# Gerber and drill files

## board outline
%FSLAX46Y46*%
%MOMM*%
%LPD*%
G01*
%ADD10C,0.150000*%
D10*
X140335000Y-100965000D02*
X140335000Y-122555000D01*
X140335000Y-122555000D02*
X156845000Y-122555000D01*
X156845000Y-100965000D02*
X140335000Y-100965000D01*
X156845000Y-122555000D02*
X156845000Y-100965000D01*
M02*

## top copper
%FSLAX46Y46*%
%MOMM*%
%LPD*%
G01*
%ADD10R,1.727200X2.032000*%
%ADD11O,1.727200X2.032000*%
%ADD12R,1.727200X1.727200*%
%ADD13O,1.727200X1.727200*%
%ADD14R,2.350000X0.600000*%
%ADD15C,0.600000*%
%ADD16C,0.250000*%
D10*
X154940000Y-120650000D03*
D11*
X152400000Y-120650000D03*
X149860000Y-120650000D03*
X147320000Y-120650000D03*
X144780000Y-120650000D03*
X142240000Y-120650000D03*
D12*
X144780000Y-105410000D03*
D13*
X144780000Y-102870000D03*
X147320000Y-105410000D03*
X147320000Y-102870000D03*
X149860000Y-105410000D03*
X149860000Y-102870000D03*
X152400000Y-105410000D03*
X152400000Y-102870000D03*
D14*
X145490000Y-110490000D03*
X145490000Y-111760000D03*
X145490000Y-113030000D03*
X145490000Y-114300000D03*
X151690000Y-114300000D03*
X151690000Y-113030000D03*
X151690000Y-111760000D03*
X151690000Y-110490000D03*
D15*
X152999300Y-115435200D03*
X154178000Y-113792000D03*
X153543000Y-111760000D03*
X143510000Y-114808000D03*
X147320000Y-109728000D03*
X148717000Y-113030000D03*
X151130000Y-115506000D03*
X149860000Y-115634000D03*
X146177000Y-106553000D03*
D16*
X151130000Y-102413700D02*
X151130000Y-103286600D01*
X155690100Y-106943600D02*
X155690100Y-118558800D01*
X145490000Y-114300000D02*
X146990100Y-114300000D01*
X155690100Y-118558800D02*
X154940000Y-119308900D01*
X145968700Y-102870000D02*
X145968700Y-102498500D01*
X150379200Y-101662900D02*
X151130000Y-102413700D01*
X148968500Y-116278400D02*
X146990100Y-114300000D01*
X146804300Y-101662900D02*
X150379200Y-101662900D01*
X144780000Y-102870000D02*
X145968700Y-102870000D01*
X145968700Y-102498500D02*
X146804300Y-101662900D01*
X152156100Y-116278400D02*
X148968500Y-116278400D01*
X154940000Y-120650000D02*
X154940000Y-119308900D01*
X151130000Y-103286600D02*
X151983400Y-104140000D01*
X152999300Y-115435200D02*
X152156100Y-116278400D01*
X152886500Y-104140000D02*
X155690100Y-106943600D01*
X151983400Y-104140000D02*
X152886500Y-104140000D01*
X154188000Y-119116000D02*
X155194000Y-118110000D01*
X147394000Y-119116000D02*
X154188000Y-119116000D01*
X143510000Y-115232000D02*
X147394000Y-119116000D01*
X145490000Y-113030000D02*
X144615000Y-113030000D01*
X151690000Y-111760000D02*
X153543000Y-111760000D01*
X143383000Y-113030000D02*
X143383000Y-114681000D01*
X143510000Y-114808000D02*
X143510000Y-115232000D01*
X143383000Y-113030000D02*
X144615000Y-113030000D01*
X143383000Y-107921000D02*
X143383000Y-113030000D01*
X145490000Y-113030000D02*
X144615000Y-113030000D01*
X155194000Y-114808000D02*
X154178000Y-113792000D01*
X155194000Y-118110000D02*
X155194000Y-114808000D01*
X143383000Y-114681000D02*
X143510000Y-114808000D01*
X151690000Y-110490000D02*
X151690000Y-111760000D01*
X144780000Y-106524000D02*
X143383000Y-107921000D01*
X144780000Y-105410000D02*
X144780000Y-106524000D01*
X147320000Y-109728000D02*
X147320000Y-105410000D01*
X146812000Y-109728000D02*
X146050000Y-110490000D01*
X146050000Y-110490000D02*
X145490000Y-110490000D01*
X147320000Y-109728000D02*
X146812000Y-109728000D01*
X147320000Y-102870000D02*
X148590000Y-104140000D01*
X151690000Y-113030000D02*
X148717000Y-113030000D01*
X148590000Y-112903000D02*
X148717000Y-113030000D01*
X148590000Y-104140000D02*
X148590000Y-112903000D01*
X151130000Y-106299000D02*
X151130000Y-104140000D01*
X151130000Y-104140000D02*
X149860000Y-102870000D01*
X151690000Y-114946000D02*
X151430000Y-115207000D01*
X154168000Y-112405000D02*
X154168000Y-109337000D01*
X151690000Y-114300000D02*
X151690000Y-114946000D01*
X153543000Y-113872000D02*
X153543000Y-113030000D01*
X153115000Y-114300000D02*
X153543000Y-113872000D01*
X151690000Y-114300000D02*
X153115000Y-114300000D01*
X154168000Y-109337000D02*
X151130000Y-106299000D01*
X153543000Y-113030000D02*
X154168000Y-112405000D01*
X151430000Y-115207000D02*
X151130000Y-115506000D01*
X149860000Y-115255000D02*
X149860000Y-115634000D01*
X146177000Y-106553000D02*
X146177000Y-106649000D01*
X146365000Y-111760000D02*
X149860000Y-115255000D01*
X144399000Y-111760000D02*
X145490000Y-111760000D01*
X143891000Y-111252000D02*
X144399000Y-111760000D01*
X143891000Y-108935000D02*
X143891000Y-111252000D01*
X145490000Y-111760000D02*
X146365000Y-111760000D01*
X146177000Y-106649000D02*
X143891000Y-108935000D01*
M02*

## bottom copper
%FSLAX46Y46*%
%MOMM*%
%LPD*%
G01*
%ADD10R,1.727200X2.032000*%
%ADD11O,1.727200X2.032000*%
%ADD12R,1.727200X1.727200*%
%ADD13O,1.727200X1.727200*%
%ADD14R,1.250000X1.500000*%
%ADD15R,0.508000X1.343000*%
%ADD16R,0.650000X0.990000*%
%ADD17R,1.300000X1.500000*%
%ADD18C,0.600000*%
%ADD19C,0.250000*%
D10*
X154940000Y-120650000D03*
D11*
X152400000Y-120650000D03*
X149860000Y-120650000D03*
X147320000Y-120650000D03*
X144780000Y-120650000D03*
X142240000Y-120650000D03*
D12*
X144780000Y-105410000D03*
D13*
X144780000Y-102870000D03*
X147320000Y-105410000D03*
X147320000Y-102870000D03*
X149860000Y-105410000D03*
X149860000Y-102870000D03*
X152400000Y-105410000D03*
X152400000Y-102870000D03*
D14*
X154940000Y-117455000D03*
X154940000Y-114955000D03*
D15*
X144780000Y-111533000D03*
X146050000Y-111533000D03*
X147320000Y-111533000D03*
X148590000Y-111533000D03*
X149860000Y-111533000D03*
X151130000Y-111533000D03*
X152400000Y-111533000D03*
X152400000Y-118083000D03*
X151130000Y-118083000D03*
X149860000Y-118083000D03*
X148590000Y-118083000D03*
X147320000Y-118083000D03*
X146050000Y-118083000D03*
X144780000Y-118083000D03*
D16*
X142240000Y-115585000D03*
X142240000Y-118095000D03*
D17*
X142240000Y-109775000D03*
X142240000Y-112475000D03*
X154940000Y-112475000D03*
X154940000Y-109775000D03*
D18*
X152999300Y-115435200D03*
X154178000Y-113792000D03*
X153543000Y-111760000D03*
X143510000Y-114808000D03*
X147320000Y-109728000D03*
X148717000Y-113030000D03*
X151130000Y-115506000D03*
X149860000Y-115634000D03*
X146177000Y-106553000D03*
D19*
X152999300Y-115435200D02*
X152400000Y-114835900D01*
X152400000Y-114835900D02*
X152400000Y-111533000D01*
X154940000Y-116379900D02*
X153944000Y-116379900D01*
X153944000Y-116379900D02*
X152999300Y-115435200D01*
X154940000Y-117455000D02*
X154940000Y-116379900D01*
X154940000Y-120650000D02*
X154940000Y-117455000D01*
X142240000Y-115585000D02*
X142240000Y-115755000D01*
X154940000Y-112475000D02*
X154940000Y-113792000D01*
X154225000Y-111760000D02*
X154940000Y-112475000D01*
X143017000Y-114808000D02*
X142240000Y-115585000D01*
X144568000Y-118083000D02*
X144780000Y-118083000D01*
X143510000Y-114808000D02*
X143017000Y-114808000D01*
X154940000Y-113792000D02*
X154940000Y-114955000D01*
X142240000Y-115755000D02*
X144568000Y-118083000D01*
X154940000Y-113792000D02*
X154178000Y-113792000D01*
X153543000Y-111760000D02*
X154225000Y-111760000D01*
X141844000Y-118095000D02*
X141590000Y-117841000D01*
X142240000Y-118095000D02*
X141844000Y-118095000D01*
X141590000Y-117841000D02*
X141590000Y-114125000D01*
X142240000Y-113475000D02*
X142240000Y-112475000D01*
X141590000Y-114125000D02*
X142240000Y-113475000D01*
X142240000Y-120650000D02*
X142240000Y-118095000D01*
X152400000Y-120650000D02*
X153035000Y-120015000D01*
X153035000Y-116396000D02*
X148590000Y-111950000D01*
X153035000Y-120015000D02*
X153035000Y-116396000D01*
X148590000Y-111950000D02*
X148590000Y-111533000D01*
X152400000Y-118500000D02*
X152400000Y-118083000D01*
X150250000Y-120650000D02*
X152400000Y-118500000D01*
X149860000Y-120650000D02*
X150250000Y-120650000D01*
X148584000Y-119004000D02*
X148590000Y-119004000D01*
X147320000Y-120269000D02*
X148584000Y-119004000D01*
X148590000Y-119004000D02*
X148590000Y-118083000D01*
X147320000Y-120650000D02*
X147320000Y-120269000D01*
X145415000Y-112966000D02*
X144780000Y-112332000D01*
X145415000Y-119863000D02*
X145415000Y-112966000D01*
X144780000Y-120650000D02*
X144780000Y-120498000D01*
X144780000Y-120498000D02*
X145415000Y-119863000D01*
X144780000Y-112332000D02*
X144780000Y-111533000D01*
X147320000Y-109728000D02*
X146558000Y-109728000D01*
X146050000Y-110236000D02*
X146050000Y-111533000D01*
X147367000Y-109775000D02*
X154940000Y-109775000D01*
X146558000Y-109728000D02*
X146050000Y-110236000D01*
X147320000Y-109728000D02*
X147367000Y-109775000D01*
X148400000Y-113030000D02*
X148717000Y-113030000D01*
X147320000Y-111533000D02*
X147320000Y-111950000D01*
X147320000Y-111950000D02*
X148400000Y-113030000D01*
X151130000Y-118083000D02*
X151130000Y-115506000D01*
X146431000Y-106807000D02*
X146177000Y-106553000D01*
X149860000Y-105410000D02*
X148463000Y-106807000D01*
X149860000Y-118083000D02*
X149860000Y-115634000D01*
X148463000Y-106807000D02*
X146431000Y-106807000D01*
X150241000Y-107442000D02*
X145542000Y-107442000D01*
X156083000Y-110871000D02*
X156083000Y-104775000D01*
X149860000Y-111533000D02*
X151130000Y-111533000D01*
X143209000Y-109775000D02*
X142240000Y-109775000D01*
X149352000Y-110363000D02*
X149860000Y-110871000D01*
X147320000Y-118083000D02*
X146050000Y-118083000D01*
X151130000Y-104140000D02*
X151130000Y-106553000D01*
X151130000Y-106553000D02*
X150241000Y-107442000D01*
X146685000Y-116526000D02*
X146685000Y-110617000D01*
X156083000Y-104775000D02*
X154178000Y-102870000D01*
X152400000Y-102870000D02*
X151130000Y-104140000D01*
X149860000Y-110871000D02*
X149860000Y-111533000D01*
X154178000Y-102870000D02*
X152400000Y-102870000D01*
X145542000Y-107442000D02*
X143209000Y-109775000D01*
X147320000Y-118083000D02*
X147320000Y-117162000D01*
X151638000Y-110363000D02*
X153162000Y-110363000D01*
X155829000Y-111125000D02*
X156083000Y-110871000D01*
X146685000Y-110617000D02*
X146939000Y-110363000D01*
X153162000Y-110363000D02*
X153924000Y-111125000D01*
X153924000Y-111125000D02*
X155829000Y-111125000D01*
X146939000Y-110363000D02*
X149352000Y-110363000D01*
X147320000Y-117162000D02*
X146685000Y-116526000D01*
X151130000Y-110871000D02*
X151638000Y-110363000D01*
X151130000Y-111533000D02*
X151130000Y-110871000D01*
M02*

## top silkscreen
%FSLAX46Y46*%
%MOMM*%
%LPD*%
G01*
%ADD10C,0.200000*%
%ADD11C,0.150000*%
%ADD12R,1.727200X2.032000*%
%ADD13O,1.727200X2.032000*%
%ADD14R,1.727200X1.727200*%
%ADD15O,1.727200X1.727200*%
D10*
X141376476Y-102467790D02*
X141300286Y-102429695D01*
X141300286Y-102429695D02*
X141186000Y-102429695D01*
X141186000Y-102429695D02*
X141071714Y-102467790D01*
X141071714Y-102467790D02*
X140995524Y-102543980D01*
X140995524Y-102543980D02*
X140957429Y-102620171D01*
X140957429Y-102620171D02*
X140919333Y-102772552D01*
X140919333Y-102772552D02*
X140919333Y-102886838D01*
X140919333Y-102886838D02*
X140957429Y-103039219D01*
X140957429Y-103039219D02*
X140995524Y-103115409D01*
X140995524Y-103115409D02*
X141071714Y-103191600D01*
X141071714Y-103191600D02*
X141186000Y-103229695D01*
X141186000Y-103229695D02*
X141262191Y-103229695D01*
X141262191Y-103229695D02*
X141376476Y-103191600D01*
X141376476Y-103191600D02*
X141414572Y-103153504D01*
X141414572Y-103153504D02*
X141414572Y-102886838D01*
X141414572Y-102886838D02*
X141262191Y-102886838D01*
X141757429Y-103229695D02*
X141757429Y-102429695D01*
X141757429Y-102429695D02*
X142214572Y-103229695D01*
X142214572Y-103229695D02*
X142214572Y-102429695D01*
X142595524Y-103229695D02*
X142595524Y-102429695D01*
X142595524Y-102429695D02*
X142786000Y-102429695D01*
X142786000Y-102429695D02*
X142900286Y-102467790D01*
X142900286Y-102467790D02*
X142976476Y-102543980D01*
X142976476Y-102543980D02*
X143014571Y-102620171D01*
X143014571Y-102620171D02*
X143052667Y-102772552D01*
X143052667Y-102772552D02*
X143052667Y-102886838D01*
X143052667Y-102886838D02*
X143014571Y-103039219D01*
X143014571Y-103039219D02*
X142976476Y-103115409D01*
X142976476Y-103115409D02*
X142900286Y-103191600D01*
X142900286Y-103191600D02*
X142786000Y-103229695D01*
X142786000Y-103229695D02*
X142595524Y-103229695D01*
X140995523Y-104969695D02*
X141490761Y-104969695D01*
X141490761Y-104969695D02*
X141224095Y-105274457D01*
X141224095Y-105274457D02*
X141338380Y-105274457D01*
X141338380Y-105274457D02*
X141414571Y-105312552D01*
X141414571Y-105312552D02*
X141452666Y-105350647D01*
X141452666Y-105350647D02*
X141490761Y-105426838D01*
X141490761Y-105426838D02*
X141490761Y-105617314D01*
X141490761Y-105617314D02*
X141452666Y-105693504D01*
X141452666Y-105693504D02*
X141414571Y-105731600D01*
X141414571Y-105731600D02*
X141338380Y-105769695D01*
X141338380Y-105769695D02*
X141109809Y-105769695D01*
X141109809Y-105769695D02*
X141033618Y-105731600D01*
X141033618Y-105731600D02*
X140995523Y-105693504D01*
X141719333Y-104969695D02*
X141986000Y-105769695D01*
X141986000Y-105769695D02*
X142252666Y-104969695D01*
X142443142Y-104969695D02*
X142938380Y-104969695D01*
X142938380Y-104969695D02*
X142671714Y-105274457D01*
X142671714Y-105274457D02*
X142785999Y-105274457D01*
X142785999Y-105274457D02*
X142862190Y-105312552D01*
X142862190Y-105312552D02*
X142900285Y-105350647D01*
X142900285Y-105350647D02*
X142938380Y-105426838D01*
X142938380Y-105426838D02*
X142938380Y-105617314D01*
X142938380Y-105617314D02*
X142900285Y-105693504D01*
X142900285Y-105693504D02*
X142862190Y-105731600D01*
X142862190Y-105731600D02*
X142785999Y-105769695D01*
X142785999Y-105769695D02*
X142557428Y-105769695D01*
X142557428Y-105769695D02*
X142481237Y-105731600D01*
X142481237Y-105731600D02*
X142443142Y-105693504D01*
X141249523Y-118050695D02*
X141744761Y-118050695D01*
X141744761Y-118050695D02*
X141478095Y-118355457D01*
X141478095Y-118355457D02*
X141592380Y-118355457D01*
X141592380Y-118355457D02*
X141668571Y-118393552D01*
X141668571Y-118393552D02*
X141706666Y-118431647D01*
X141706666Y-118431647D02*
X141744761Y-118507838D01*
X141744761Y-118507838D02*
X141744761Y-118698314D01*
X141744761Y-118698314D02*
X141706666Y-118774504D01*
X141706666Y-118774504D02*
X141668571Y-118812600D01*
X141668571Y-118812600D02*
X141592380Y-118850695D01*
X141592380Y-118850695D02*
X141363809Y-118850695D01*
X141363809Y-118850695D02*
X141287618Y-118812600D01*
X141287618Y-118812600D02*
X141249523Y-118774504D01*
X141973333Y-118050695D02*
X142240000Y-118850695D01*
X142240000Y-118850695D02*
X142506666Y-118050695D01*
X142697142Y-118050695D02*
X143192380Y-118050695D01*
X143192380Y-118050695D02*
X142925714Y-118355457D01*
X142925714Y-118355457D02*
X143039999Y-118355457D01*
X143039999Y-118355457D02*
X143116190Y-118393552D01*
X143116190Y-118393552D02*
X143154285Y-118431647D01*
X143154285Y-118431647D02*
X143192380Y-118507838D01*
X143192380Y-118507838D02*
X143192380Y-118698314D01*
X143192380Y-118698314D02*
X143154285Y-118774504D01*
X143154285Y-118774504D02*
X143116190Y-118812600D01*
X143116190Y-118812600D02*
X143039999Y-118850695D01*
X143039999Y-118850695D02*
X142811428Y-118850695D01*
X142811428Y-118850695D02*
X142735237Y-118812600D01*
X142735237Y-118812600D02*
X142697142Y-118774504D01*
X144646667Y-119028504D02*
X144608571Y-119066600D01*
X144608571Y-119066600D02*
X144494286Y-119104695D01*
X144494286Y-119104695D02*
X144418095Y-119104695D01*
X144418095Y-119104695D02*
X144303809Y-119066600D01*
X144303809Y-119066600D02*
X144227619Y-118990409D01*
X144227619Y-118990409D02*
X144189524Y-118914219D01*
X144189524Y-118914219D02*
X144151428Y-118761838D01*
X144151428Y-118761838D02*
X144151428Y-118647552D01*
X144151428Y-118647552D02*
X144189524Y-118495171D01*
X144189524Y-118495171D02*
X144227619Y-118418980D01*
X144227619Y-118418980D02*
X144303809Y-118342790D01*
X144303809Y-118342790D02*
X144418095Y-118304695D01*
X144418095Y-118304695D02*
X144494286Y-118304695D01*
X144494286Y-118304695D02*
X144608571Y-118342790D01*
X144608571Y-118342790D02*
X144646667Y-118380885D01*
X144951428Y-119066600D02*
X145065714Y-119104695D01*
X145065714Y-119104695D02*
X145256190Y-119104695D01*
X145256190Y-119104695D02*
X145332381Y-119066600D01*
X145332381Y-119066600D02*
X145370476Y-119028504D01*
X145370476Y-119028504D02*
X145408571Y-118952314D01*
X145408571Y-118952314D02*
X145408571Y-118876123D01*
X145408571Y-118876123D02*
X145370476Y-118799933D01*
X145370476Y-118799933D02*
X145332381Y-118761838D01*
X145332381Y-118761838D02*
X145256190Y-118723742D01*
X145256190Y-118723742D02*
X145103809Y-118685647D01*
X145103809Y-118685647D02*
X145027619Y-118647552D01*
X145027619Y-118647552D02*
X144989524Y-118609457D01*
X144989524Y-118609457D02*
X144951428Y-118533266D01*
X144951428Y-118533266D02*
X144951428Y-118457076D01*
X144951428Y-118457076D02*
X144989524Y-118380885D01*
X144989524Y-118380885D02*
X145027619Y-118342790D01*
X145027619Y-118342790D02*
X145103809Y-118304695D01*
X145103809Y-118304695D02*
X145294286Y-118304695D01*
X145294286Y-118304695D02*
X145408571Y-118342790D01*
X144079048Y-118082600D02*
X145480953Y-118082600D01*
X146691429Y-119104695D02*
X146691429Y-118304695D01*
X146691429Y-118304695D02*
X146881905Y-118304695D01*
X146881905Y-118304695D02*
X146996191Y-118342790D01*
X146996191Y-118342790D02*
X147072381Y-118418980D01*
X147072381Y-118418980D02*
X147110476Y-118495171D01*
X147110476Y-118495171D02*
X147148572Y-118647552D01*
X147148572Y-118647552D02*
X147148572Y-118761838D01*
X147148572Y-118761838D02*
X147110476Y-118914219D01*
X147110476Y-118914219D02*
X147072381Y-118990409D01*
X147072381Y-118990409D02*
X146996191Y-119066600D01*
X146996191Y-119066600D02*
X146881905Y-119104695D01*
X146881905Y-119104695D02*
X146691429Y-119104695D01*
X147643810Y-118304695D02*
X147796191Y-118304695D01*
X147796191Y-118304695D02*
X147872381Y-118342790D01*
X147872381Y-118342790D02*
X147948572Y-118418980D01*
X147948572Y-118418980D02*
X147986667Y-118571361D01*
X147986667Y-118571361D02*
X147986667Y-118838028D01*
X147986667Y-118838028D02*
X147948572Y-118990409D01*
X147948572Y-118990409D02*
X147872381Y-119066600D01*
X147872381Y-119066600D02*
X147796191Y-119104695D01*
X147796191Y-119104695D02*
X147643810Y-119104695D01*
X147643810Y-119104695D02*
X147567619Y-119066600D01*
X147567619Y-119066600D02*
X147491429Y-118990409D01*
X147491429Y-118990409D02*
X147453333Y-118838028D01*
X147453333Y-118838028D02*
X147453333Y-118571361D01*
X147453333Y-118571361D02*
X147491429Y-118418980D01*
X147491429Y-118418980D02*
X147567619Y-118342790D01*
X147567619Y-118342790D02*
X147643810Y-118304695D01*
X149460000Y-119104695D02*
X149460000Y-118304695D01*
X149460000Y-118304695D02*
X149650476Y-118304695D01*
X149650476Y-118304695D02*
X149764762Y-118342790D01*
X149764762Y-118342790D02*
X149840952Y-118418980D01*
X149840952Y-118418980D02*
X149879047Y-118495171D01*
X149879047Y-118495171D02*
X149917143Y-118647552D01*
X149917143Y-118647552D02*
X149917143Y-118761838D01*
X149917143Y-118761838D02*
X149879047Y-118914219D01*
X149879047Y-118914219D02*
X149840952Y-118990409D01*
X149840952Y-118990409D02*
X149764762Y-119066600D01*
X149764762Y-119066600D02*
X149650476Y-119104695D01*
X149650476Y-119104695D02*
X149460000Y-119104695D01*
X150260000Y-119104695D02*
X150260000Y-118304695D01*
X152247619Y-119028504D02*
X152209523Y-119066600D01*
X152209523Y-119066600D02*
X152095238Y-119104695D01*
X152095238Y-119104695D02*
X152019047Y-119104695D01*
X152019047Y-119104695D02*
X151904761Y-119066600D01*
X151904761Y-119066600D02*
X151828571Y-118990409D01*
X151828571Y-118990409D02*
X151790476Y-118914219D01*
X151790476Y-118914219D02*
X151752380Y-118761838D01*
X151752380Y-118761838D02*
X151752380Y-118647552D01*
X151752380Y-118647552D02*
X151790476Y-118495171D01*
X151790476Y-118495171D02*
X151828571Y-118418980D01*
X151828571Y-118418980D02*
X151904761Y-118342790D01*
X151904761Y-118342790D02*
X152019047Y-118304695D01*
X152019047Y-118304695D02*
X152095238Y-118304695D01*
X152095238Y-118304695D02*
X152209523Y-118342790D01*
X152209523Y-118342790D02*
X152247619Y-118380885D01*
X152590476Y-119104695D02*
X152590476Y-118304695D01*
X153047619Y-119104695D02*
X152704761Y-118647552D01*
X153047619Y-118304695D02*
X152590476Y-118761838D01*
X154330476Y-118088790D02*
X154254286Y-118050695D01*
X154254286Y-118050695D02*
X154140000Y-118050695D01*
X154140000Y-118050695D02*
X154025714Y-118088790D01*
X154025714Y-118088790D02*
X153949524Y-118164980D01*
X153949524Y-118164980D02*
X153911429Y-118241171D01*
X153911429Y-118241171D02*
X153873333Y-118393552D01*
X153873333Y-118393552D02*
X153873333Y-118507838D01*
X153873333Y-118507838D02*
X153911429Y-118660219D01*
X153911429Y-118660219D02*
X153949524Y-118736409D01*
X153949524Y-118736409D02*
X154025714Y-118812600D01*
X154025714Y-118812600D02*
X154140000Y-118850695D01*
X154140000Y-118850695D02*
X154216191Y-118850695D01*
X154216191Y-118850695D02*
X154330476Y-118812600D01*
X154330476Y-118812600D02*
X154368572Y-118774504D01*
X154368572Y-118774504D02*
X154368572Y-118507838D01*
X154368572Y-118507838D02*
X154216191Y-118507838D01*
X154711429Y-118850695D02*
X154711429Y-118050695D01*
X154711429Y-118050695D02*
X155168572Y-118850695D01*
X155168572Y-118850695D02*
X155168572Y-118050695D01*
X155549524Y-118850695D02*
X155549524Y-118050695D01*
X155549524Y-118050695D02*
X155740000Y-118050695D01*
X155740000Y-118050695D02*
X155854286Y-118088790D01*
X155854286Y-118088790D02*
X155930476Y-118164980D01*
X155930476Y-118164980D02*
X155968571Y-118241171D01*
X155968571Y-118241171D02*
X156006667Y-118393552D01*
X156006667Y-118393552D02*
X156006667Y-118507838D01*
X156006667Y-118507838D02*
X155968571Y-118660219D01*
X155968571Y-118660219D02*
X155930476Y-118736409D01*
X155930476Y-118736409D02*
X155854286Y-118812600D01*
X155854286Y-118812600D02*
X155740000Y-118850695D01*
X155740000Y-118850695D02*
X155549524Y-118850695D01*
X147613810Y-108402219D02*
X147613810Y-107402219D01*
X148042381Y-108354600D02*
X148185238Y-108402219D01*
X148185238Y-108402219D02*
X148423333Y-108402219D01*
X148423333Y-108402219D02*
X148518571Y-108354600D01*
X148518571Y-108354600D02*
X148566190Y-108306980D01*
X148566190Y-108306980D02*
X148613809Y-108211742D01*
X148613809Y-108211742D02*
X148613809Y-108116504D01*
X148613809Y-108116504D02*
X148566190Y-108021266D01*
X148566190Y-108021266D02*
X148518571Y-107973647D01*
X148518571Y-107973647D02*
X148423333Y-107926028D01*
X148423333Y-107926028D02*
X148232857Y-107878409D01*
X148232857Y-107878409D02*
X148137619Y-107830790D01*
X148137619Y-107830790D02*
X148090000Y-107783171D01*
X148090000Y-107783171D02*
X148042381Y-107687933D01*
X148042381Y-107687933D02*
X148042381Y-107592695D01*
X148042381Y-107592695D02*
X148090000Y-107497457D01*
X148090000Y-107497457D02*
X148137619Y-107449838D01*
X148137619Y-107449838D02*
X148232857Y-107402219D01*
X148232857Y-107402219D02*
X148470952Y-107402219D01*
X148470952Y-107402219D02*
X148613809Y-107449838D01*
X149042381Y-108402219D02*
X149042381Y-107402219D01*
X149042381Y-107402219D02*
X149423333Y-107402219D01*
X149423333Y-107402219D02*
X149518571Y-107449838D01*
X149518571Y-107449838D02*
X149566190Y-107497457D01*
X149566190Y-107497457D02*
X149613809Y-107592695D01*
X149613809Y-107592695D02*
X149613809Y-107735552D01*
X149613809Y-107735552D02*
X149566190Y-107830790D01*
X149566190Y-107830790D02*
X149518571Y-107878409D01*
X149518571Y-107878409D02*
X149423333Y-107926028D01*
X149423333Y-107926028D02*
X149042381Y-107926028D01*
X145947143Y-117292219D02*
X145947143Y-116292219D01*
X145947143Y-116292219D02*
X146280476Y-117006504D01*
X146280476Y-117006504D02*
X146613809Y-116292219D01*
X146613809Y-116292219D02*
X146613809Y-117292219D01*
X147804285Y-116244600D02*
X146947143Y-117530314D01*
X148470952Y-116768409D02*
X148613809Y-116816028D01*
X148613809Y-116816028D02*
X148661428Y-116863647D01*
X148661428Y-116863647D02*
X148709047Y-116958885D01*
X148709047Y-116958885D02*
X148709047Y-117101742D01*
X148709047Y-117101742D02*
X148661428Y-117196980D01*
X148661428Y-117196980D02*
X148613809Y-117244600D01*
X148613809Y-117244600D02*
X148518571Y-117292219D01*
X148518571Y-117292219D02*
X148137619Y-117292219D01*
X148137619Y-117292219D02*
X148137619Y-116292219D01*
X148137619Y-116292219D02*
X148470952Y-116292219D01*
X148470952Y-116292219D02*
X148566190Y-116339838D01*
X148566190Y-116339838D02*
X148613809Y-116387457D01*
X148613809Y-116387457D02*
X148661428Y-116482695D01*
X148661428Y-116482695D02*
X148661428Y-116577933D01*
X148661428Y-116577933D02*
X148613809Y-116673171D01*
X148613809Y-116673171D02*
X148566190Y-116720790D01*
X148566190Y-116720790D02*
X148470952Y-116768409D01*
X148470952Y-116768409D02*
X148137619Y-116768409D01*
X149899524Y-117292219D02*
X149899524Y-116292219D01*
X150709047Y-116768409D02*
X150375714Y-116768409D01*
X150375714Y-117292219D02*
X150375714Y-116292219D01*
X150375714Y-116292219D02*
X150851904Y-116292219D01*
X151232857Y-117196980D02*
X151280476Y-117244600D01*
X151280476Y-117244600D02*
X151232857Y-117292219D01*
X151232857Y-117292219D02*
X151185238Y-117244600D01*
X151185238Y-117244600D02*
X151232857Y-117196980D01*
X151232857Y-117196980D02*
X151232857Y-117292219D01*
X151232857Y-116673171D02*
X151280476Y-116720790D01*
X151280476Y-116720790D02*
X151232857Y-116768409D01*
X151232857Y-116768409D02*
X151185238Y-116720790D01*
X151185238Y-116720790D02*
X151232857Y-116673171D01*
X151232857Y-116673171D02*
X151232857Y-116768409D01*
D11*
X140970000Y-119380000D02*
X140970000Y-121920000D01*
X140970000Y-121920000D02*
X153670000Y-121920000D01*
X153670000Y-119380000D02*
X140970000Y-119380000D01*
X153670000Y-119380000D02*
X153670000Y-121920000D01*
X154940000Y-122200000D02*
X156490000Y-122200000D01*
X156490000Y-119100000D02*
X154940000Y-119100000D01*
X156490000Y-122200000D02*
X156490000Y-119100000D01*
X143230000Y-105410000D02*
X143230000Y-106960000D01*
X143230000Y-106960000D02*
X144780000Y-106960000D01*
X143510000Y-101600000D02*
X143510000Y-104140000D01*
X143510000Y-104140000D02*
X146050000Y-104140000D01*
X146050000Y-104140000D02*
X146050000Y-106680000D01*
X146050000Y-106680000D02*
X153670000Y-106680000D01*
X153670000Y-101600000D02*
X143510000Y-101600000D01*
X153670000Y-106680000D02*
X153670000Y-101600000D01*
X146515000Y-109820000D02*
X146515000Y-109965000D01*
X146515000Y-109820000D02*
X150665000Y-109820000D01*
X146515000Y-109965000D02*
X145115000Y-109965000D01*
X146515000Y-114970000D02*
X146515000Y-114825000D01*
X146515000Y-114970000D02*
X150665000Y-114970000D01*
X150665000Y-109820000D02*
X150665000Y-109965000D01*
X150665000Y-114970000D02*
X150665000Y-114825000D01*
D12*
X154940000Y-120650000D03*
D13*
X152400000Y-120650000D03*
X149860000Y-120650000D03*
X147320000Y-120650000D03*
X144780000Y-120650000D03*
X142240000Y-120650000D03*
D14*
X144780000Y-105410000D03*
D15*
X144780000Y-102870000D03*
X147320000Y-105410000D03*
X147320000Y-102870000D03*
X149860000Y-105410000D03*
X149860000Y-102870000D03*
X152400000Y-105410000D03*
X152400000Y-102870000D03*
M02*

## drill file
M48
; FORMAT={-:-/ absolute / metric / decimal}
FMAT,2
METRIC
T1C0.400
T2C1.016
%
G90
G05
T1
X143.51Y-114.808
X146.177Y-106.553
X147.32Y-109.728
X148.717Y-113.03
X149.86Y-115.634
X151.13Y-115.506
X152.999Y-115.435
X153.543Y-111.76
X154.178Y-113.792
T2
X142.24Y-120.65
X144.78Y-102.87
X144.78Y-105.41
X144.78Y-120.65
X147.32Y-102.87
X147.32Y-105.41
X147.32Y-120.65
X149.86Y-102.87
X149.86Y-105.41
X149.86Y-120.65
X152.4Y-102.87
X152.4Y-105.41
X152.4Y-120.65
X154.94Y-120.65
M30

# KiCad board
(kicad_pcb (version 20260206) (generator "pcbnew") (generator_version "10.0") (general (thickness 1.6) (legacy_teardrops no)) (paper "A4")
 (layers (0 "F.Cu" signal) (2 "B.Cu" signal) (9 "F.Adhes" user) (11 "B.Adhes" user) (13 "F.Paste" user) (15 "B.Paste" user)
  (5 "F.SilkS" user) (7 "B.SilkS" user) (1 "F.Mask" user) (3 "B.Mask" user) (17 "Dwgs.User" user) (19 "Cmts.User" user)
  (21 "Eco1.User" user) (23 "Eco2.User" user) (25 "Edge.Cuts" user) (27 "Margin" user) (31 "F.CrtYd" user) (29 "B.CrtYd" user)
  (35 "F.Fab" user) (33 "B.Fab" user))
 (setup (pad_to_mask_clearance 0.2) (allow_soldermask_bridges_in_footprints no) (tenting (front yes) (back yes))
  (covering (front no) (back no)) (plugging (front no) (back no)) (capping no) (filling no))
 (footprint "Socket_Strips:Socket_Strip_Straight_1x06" (layer "F.Cu") (at 154.94 120.65 180)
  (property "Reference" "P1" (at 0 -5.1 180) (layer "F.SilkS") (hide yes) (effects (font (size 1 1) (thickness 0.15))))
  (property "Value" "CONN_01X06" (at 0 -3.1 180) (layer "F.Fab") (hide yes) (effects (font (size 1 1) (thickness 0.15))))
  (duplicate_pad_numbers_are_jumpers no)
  (fp_line (start 13.97 1.27) (end 13.97 -1.27) (stroke (width 0.15) (type solid)) (layer "F.SilkS"))
  (fp_line (start 13.97 -1.27) (end 1.27 -1.27) (stroke (width 0.15) (type solid)) (layer "F.SilkS"))
  (fp_line (start 1.27 1.27) (end 13.97 1.27) (stroke (width 0.15) (type solid)) (layer "F.SilkS"))
  (fp_line (start 1.27 1.27) (end 1.27 -1.27) (stroke (width 0.15) (type solid)) (layer "F.SilkS"))
  (fp_line (start 0 -1.55) (end -1.55 -1.55) (stroke (width 0.15) (type solid)) (layer "F.SilkS"))
  (fp_line (start -1.55 1.55) (end 0 1.55) (stroke (width 0.15) (type solid)) (layer "F.SilkS"))
  (fp_line (start -1.55 -1.55) (end -1.55 1.55) (stroke (width 0.15) (type solid)) (layer "F.SilkS"))
  (pad "1" thru_hole rect (at 0 0 180) (size 1.7272 2.032) (drill 1.016) (layers "*.Cu" "*.Mask" "F.SilkS") (remove_unused_layers no)
   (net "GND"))
  (pad "2" thru_hole oval (at 2.54 0 180) (size 1.7272 2.032) (drill 1.016) (layers "*.Cu" "*.Mask" "F.SilkS") (remove_unused_layers no)
   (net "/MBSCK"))
  (pad "3" thru_hole oval (at 5.08 0 180) (size 1.7272 2.032) (drill 1.016) (layers "*.Cu" "*.Mask" "F.SilkS") (remove_unused_layers no)
   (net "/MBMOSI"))
  (pad "4" thru_hole oval (at 7.62 0 180) (size 1.7272 2.032) (drill 1.016) (layers "*.Cu" "*.Mask" "F.SilkS") (remove_unused_layers no)
   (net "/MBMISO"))
  (pad "5" thru_hole oval (at 10.16 0 180) (size 1.7272 2.032) (drill 1.016) (layers "*.Cu" "*.Mask" "F.SilkS") (remove_unused_layers no)
   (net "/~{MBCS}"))
  (pad "6" thru_hole oval (at 12.7 0 180) (size 1.7272 2.032) (drill 1.016) (layers "*.Cu" "*.Mask" "F.SilkS") (remove_unused_layers no)
   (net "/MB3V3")))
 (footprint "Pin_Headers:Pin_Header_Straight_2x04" (layer "F.Cu") (at 144.78 105.41 90)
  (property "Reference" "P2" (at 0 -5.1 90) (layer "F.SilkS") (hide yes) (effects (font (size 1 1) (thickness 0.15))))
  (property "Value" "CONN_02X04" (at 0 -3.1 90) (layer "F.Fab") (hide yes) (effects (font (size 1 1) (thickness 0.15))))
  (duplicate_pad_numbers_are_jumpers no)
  (fp_line (start 0 -1.55) (end -1.55 -1.55) (stroke (width 0.15) (type solid)) (layer "F.SilkS"))
  (fp_line (start -1.55 -1.55) (end -1.55 0) (stroke (width 0.15) (type solid)) (layer "F.SilkS"))
  (fp_line (start 3.81 -1.27) (end 1.27 -1.27) (stroke (width 0.15) (type solid)) (layer "F.SilkS"))
  (fp_line (start 1.27 -1.27) (end 1.27 1.27) (stroke (width 0.15) (type solid)) (layer "F.SilkS"))
  (fp_line (start 1.27 1.27) (end -1.27 1.27) (stroke (width 0.15) (type solid)) (layer "F.SilkS"))
  (fp_line (start -1.27 1.27) (end -1.27 8.89) (stroke (width 0.15) (type solid)) (layer "F.SilkS"))
  (fp_line (start 3.81 8.89) (end 3.81 -1.27) (stroke (width 0.15) (type solid)) (layer "F.SilkS"))
  (fp_line (start -1.27 8.89) (end 3.81 8.89) (stroke (width 0.15) (type solid)) (layer "F.SilkS"))
  (pad "1" thru_hole rect (at 0 0 90) (size 1.7272 1.7272) (drill 1.016) (layers "*.Cu" "*.Mask" "F.SilkS") (remove_unused_layers no)
   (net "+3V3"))
  (pad "2" thru_hole oval (at 2.54 0 90) (size 1.7272 1.7272) (drill 1.016) (layers "*.Cu" "*.Mask" "F.SilkS") (remove_unused_layers no)
   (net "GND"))
  (pad "3" thru_hole oval (at 0 2.54 90) (size 1.7272 1.7272) (drill 1.016) (layers "*.Cu" "*.Mask" "F.SilkS") (remove_unused_layers no)
   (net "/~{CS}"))
  (pad "4" thru_hole oval (at 2.54 2.54 90) (size 1.7272 1.7272) (drill 1.016) (layers "*.Cu" "*.Mask" "F.SilkS") (remove_unused_layers no)
   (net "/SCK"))
  (pad "5" thru_hole oval (at 0 5.08 90) (size 1.7272 1.7272) (drill 1.016) (layers "*.Cu" "*.Mask" "F.SilkS") (remove_unused_layers no)
   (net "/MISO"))
  (pad "6" thru_hole oval (at 2.54 5.08 90) (size 1.7272 1.7272) (drill 1.016) (layers "*.Cu" "*.Mask" "F.SilkS") (remove_unused_layers no)
   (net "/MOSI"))
  (pad "7" thru_hole oval (at 0 7.62 90) (size 1.7272 1.7272) (drill 1.016) (layers "*.Cu" "*.Mask" "F.SilkS") (remove_unused_layers no))
  (pad "8" thru_hole oval (at 2.54 7.62 90) (size 1.7272 1.7272) (drill 1.016) (layers "*.Cu" "*.Mask" "F.SilkS") (remove_unused_layers no)
   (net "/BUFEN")))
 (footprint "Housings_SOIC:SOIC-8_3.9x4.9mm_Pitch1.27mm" (layer "F.Cu") (at 148.59 112.395)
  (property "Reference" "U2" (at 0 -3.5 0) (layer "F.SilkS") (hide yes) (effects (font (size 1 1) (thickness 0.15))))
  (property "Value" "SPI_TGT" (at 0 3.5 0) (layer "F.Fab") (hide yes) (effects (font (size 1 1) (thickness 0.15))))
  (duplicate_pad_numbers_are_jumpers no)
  (fp_line (start -2.075 -2.575) (end -2.075 -2.43) (stroke (width 0.15) (type solid)) (layer "F.SilkS"))
  (fp_line (start -2.075 -2.575) (end 2.075 -2.575) (stroke (width 0.15) (type solid)) (layer "F.SilkS"))
  (fp_line (start -2.075 -2.43) (end -3.475 -2.43) (stroke (width 0.15) (type solid)) (layer "F.SilkS"))
  (fp_line (start -2.075 2.575) (end -2.075 2.43) (stroke (width 0.15) (type solid)) (layer "F.SilkS"))
  (fp_line (start -2.075 2.575) (end 2.075 2.575) (stroke (width 0.15) (type solid)) (layer "F.SilkS"))
  (fp_line (start 2.075 -2.575) (end 2.075 -2.43) (stroke (width 0.15) (type solid)) (layer "F.SilkS"))
  (fp_line (start 2.075 2.575) (end 2.075 2.43) (stroke (width 0.15) (type solid)) (layer "F.SilkS"))
  (pad "1" smd rect (at -3.1 -1.905) (size 2.35 0.6) (layers "F.Cu" "F.Mask" "F.Paste") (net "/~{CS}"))
  (pad "2" smd rect (at -3.1 -0.635) (size 2.35 0.6) (layers "F.Cu" "F.Mask" "F.Paste") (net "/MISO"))
  (pad "3" smd rect (at -3.1 0.635) (size 2.35 0.6) (layers "F.Cu" "F.Mask" "F.Paste") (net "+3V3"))
  (pad "4" smd rect (at -3.1 1.905) (size 2.35 0.6) (layers "F.Cu" "F.Mask" "F.Paste") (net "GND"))
  (pad "5" smd rect (at 3.1 1.905) (size 2.35 0.6) (layers "F.Cu" "F.Mask" "F.Paste") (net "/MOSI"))
  (pad "6" smd rect (at 3.1 0.635) (size 2.35 0.6) (layers "F.Cu" "F.Mask" "F.Paste") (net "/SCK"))
  (pad "7" smd rect (at 3.1 -0.635) (size 2.35 0.6) (layers "F.Cu" "F.Mask" "F.Paste") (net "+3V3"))
  (pad "8" smd rect (at 3.1 -1.905) (size 2.35 0.6) (layers "F.Cu" "F.Mask" "F.Paste") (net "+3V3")))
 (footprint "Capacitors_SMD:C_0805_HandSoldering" (layer "B.Cu") (at 154.94 116.205 90)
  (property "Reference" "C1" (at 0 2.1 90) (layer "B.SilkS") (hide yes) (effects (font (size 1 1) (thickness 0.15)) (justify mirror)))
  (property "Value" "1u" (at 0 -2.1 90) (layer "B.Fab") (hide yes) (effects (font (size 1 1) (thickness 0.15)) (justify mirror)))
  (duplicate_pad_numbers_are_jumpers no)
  (pad "1" smd rect (at -1.25 0 90) (size 1.5 1.25) (layers "B.Cu" "B.Mask" "B.Paste") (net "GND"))
  (pad "2" smd rect (at 1.25 0 90) (size 1.5 1.25) (layers "B.Cu" "B.Mask" "B.Paste") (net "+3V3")))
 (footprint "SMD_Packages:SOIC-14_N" (layer "B.Cu") (at 148.59 114.935)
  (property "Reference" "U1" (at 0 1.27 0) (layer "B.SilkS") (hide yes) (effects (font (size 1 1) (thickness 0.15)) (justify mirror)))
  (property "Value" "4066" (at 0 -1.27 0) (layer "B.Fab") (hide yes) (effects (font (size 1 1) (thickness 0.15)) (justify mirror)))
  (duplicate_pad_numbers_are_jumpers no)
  (pad "1" smd rect (at -3.81 -3.402) (size 0.508 1.343) (layers "B.Cu" "B.Mask" "B.Paste") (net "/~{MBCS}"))
  (pad "2" smd rect (at -2.54 -3.402) (size 0.508 1.343) (layers "B.Cu" "B.Mask" "B.Paste") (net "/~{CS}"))
  (pad "3" smd rect (at -1.27 -3.402) (size 0.508 1.343) (layers "B.Cu" "B.Mask" "B.Paste") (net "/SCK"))
  (pad "4" smd rect (at 0 -3.402) (size 0.508 1.343) (layers "B.Cu" "B.Mask" "B.Paste") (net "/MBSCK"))
  (pad "5" smd rect (at 1.27 -3.402) (size 0.508 1.343) (layers "B.Cu" "B.Mask" "B.Paste") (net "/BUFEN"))
  (pad "6" smd rect (at 2.54 -3.402) (size 0.508 1.343) (layers "B.Cu" "B.Mask" "B.Paste") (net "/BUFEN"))
  (pad "7" smd rect (at 3.81 -3.402) (size 0.508 1.343) (layers "B.Cu" "B.Mask" "B.Paste") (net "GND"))
  (pad "8" smd rect (at 3.81 3.148) (size 0.508 1.343) (layers "B.Cu" "B.Mask" "B.Paste") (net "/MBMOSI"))
  (pad "9" smd rect (at 2.54 3.148) (size 0.508 1.343) (layers "B.Cu" "B.Mask" "B.Paste") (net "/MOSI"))
  (pad "10" smd rect (at 1.27 3.148 180) (size 0.508 1.343) (layers "B.Cu" "B.Mask" "B.Paste") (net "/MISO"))
  (pad "11" smd rect (at 0 3.148) (size 0.508 1.343) (layers "B.Cu" "B.Mask" "B.Paste") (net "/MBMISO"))
  (pad "12" smd rect (at -1.27 3.148) (size 0.508 1.343) (layers "B.Cu" "B.Mask" "B.Paste") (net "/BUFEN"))
  (pad "13" smd rect (at -2.54 3.148) (size 0.508 1.343) (layers "B.Cu" "B.Mask" "B.Paste") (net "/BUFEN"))
  (pad "14" smd rect (at -3.81 3.148) (size 0.508 1.343) (layers "B.Cu" "B.Mask" "B.Paste") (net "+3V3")))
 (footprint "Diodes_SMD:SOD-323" (layer "B.Cu") (at 142.24 116.84 -90)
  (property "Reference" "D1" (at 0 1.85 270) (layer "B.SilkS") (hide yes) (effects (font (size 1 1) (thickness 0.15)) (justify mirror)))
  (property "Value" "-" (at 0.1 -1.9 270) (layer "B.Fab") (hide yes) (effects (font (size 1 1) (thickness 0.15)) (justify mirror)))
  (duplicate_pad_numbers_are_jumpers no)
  (pad "1" smd rect (at -1.255 0 270) (size 0.99 0.65) (layers "B.Cu" "B.Mask" "B.Paste") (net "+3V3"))
  (pad "2" smd rect (at 1.255 0 270) (size 0.99 0.65) (layers "B.Cu" "B.Mask" "B.Paste") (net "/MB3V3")))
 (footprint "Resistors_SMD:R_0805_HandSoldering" (layer "B.Cu") (at 142.24 111.125 -90)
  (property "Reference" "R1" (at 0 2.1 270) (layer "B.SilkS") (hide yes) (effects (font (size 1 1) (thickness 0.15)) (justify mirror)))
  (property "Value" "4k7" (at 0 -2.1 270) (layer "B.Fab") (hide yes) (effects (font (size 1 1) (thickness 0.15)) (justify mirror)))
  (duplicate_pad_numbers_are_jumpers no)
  (pad "1" smd rect (at -1.35 0 270) (size 1.5 1.3) (layers "B.Cu" "B.Mask" "B.Paste") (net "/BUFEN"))
  (pad "2" smd rect (at 1.35 0 270) (size 1.5 1.3) (layers "B.Cu" "B.Mask" "B.Paste") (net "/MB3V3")))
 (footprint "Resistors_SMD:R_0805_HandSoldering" (layer "B.Cu") (at 154.94 111.125 90)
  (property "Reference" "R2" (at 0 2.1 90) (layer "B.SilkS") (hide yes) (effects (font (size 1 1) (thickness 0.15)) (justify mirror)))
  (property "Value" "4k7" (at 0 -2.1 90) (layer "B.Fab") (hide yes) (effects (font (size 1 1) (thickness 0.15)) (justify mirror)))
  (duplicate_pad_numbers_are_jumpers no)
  (pad "1" smd rect (at -1.35 0 90) (size 1.5 1.3) (layers "B.Cu" "B.Mask" "B.Paste") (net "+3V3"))
  (pad "2" smd rect (at 1.35 0 90) (size 1.5 1.3) (layers "B.Cu" "B.Mask" "B.Paste") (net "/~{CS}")))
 (gr_line (start 140.335 100.965) (end 140.335 122.555) (stroke (width 0.15) (type solid)) (layer "Edge.Cuts"))
 (gr_line (start 140.335 122.555) (end 156.845 122.555) (stroke (width 0.15) (type solid)) (layer "Edge.Cuts"))
 (gr_line (start 156.845 100.965) (end 140.335 100.965) (stroke (width 0.15) (type solid)) (layer "Edge.Cuts"))
 (gr_line (start 156.845 122.555) (end 156.845 100.965) (stroke (width 0.15) (type solid)) (layer "Edge.Cuts"))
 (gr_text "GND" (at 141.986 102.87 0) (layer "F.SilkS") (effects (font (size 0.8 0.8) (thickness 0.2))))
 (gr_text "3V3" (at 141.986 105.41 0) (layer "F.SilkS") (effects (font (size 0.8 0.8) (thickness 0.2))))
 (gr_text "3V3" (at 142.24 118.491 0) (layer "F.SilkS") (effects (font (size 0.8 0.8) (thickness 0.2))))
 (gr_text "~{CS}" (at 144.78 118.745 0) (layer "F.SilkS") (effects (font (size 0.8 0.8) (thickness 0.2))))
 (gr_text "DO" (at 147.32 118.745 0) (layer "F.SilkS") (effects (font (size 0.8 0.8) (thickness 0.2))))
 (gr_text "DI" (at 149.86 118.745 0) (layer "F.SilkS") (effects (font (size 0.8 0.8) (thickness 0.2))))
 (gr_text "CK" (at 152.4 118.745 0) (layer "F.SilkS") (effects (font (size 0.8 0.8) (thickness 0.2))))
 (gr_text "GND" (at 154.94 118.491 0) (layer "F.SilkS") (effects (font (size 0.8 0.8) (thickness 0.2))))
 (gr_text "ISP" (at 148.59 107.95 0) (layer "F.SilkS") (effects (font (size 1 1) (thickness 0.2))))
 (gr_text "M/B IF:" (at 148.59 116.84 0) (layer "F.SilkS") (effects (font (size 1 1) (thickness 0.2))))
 (segment (start 151.13 102.4137) (end 151.13 103.2866) (width 0.25) (layer "F.Cu") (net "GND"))
 (segment (start 155.6901 106.9436) (end 155.6901 118.5588) (width 0.25) (layer "F.Cu") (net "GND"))
 (segment (start 145.49 114.3) (end 146.9901 114.3) (width 0.25) (layer "F.Cu") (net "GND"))
 (segment (start 155.6901 118.5588) (end 154.94 119.3089) (width 0.25) (layer "F.Cu") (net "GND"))
 (segment (start 145.9687 102.87) (end 145.9687 102.4985) (width 0.25) (layer "F.Cu") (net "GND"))
 (segment (start 150.3792 101.6629) (end 151.13 102.4137) (width 0.25) (layer "F.Cu") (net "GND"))
 (segment (start 148.9685 116.2784) (end 146.9901 114.3) (width 0.25) (layer "F.Cu") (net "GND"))
 (segment (start 146.8043 101.6629) (end 150.3792 101.6629) (width 0.25) (layer "F.Cu") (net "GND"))
 (segment (start 144.78 102.87) (end 145.9687 102.87) (width 0.25) (layer "F.Cu") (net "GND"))
 (segment (start 145.9687 102.4985) (end 146.8043 101.6629) (width 0.25) (layer "F.Cu") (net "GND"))
 (segment (start 152.1561 116.2784) (end 148.9685 116.2784) (width 0.25) (layer "F.Cu") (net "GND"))
 (segment (start 154.94 120.65) (end 154.94 119.3089) (width 0.25) (layer "F.Cu") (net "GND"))
 (segment (start 151.13 103.2866) (end 151.9834 104.14) (width 0.25) (layer "F.Cu") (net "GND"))
 (segment (start 152.9993 115.4352) (end 152.1561 116.2784) (width 0.25) (layer "F.Cu") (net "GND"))
 (segment (start 152.8865 104.14) (end 155.6901 106.9436) (width 0.25) (layer "F.Cu") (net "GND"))
 (segment (start 151.9834 104.14) (end 152.8865 104.14) (width 0.25) (layer "F.Cu") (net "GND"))
 (via (at 152.9993 115.4352) (size 0.6) (drill 0.4) (layers "F.Cu" "B.Cu") (capping no) (covering (front no) (back no))
  (plugging (front no) (back no)) (filling no) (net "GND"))
 (segment (start 152.9993 115.4352) (end 152.4 114.8359) (width 0.25) (layer "B.Cu") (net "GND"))
 (segment (start 152.4 114.8359) (end 152.4 111.533) (width 0.25) (layer "B.Cu") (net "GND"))
 (segment (start 154.94 116.3799) (end 153.944 116.3799) (width 0.25) (layer "B.Cu") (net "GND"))
 (segment (start 153.944 116.3799) (end 152.9993 115.4352) (width 0.25) (layer "B.Cu") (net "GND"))
 (segment (start 154.94 117.455) (end 154.94 116.3799) (width 0.25) (layer "B.Cu") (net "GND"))
 (segment (start 154.94 120.65) (end 154.94 117.455) (width 0.25) (layer "B.Cu") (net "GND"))
 (segment (start 154.188 119.116) (end 155.194 118.11) (width 0.25) (layer "F.Cu") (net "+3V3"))
 (segment (start 147.394 119.116) (end 154.188 119.116) (width 0.25) (layer "F.Cu") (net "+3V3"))
 (segment (start 143.51 115.232) (end 147.394 119.116) (width 0.25) (layer "F.Cu") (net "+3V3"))
 (segment (start 145.49 113.03) (end 144.615 113.03) (width 0.25) (layer "F.Cu") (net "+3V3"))
 (segment (start 151.69 111.76) (end 153.543 111.76) (width 0.25) (layer "F.Cu") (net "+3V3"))
 (segment (start 143.383 113.03) (end 143.383 114.681) (width 0.25) (layer "F.Cu") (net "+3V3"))
 (segment (start 143.51 114.808) (end 143.51 115.232) (width 0.25) (layer "F.Cu") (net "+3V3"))
 (segment (start 143.383 113.03) (end 144.615 113.03) (width 0.25) (layer "F.Cu") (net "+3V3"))
 (segment (start 143.383 107.921) (end 143.383 113.03) (width 0.25) (layer "F.Cu") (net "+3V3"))
 (segment (start 145.49 113.03) (end 144.615 113.03) (width 0.25) (layer "F.Cu") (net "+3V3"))
 (segment (start 155.194 114.808) (end 154.178 113.792) (width 0.25) (layer "F.Cu") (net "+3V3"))
 (segment (start 155.194 118.11) (end 155.194 114.808) (width 0.25) (layer "F.Cu") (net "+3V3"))
 (segment (start 143.383 114.681) (end 143.51 114.808) (width 0.25) (layer "F.Cu") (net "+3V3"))
 (segment (start 151.69 110.49) (end 151.69 111.76) (width 0.25) (layer "F.Cu") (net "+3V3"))
 (segment (start 144.78 106.524) (end 143.383 107.921) (width 0.25) (layer "F.Cu") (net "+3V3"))
 (segment (start 144.78 105.41) (end 144.78 106.524) (width 0.25) (layer "F.Cu") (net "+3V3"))
 (via (at 154.178 113.792) (size 0.6) (drill 0.4) (layers "F.Cu" "B.Cu") (capping no) (covering (front no) (back no))
  (plugging (front no) (back no)) (filling no) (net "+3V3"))
 (via (at 153.543 111.76) (size 0.6) (drill 0.4) (layers "F.Cu" "B.Cu") (capping no) (covering (front no) (back no))
  (plugging (front no) (back no)) (filling no) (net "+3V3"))
 (via (at 143.51 114.808) (size 0.6) (drill 0.4) (layers "F.Cu" "B.Cu") (capping no) (covering (front no) (back no))
  (plugging (front no) (back no)) (filling no) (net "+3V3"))
 (segment (start 142.24 115.585) (end 142.24 115.755) (width 0.25) (layer "B.Cu") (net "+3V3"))
 (segment (start 154.94 112.475) (end 154.94 113.792) (width 0.25) (layer "B.Cu") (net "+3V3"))
 (segment (start 154.225 111.76) (end 154.94 112.475) (width 0.25) (layer "B.Cu") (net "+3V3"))
 (segment (start 143.017 114.808) (end 142.24 115.585) (width 0.25) (layer "B.Cu") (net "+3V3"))
 (segment (start 144.568 118.083) (end 144.78 118.083) (width 0.25) (layer "B.Cu") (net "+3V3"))
 (segment (start 143.51 114.808) (end 143.017 114.808) (width 0.25) (layer "B.Cu") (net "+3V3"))
 (segment (start 154.94 113.792) (end 154.94 114.955) (width 0.25) (layer "B.Cu") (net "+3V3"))
 (segment (start 142.24 115.755) (end 144.568 118.083) (width 0.25) (layer "B.Cu") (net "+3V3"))
 (segment (start 154.94 113.792) (end 154.178 113.792) (width 0.25) (layer "B.Cu") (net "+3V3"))
 (segment (start 153.543 111.76) (end 154.225 111.76) (width 0.25) (layer "B.Cu") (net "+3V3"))
 (segment (start 141.844 118.095) (end 141.59 117.841) (width 0.25) (layer "B.Cu") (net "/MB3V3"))
 (segment (start 142.24 118.095) (end 141.844 118.095) (width 0.25) (layer "B.Cu") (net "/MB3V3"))
 (segment (start 141.59 117.841) (end 141.59 114.125) (width 0.25) (layer "B.Cu") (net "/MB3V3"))
 (segment (start 142.24 113.475) (end 142.24 112.475) (width 0.25) (layer "B.Cu") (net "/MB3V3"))
 (segment (start 141.59 114.125) (end 142.24 113.475) (width 0.25) (layer "B.Cu") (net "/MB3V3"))
 (segment (start 142.24 120.65) (end 142.24 118.095) (width 0.25) (layer "B.Cu") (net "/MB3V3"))
 (segment (start 152.4 120.65) (end 153.035 120.015) (width 0.25) (layer "B.Cu") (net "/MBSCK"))
 (segment (start 153.035 116.396) (end 148.59 111.95) (width 0.25) (layer "B.Cu") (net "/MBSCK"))
 (segment (start 153.035 120.015) (end 153.035 116.396) (width 0.25) (layer "B.Cu") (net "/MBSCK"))
 (segment (start 148.59 111.95) (end 148.59 111.533) (width 0.25) (layer "B.Cu") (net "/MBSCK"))
 (segment (start 152.4 118.5) (end 152.4 118.083) (width 0.25) (layer "B.Cu") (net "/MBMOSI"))
 (segment (start 150.25 120.65) (end 152.4 118.5) (width 0.25) (layer "B.Cu") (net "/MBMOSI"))
 (segment (start 149.86 120.65) (end 150.25 120.65) (width 0.25) (layer "B.Cu") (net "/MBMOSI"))
 (segment (start 148.584 119.004) (end 148.59 119.004) (width 0.25) (layer "B.Cu") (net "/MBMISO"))
 (segment (start 147.32 120.269) (end 148.584 119.004) (width 0.25) (layer "B.Cu") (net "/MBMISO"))
 (segment (start 148.59 119.004) (end 148.59 118.083) (width 0.25) (layer "B.Cu") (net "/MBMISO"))
 (segment (start 147.32 120.65) (end 147.32 120.269) (width 0.25) (layer "B.Cu") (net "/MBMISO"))
 (segment (start 145.415 112.966) (end 144.78 112.332) (width 0.25) (layer "B.Cu") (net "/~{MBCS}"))
 (segment (start 145.415 119.863) (end 145.415 112.966) (width 0.25) (layer "B.Cu") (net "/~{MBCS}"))
 (segment (start 144.78 120.65) (end 144.78 120.498) (width 0.25) (layer "B.Cu") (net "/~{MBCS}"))
 (segment (start 144.78 120.498) (end 145.415 119.863) (width 0.25) (layer "B.Cu") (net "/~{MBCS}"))
 (segment (start 144.78 112.332) (end 144.78 111.533) (width 0.25) (layer "B.Cu") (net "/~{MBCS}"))
 (segment (start 147.32 109.728) (end 147.32 105.41) (width 0.25) (layer "F.Cu") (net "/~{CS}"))
 (segment (start 146.812 109.728) (end 146.05 110.49) (width 0.25) (layer "F.Cu") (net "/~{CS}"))
 (segment (start 146.05 110.49) (end 145.49 110.49) (width 0.25) (layer "F.Cu") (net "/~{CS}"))
 (segment (start 147.32 109.728) (end 146.812 109.728) (width 0.25) (layer "F.Cu") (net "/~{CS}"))
 (via (at 147.32 109.728) (size 0.6) (drill 0.4) (layers "F.Cu" "B.Cu") (capping no) (covering (front no) (back no))
  (plugging (front no) (back no)) (filling no) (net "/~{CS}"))
 (segment (start 147.32 109.728) (end 146.558 109.728) (width 0.25) (layer "B.Cu") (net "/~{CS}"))
 (segment (start 146.05 110.236) (end 146.05 111.533) (width 0.25) (layer "B.Cu") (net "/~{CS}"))
 (segment (start 147.367 109.775) (end 154.94 109.775) (width 0.25) (layer "B.Cu") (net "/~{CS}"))
 (segment (start 146.558 109.728) (end 146.05 110.236) (width 0.25) (layer "B.Cu") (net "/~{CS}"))
 (segment (start 147.32 109.728) (end 147.367 109.775) (width 0.25) (layer "B.Cu") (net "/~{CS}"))
 (segment (start 147.32 102.87) (end 148.59 104.14) (width 0.25) (layer "F.Cu") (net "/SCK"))
 (segment (start 151.69 113.03) (end 148.717 113.03) (width 0.25) (layer "F.Cu") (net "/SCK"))
 (segment (start 148.59 112.903) (end 148.717 113.03) (width 0.25) (layer "F.Cu") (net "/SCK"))
 (segment (start 148.59 104.14) (end 148.59 112.903) (width 0.25) (layer "F.Cu") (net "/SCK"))
 (via (at 148.717 113.03) (size 0.6) (drill 0.4) (layers "F.Cu" "B.Cu") (capping no) (covering (front no) (back no))
  (plugging (front no) (back no)) (filling no) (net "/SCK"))
 (segment (start 148.4 113.03) (end 148.717 113.03) (width 0.25) (layer "B.Cu") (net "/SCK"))
 (segment (start 147.32 111.533) (end 147.32 111.95) (width 0.25) (layer "B.Cu") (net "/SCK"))
 (segment (start 147.32 111.95) (end 148.4 113.03) (width 0.25) (layer "B.Cu") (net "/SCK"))
 (segment (start 151.13 106.299) (end 151.13 104.14) (width 0.25) (layer "F.Cu") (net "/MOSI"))
 (segment (start 151.13 104.14) (end 149.86 102.87) (width 0.25) (layer "F.Cu") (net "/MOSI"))
 (segment (start 151.69 114.946) (end 151.43 115.207) (width 0.25) (layer "F.Cu") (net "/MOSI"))
 (segment (start 154.168 112.405) (end 154.168 109.337) (width 0.25) (layer "F.Cu") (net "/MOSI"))
 (segment (start 151.69 114.3) (end 151.69 114.946) (width 0.25) (layer "F.Cu") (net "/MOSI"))
 (segment (start 153.543 113.872) (end 153.543 113.03) (width 0.25) (layer "F.Cu") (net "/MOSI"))
 (segment (start 153.115 114.3) (end 153.543 113.872) (width 0.25) (layer "F.Cu") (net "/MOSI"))
 (segment (start 151.69 114.3) (end 153.115 114.3) (width 0.25) (layer "F.Cu") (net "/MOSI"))
 (segment (start 154.168 109.337) (end 151.13 106.299) (width 0.25) (layer "F.Cu") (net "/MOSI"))
 (segment (start 153.543 113.03) (end 154.168 112.405) (width 0.25) (layer "F.Cu") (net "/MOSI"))
 (segment (start 151.43 115.207) (end 151.13 115.506) (width 0.25) (layer "F.Cu") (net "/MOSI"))
 (via (at 151.13 115.506) (size 0.6) (drill 0.4) (layers "F.Cu" "B.Cu") (capping no) (covering (front no) (back no))
  (plugging (front no) (back no)) (filling no) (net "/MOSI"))
 (segment (start 151.13 118.083) (end 151.13 115.506) (width 0.25) (layer "B.Cu") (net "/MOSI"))
 (segment (start 149.86 115.255) (end 149.86 115.634) (width 0.25) (layer "F.Cu") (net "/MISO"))
 (segment (start 146.177 106.553) (end 146.177 106.649) (width 0.25) (layer "F.Cu") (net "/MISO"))
 (segment (start 146.365 111.76) (end 149.86 115.255) (width 0.25) (layer "F.Cu") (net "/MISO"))
 (segment (start 144.399 111.76) (end 145.49 111.76) (width 0.25) (layer "F.Cu") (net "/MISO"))
 (segment (start 143.891 111.252) (end 144.399 111.76) (width 0.25) (layer "F.Cu") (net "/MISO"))
 (segment (start 143.891 108.935) (end 143.891 111.252) (width 0.25) (layer "F.Cu") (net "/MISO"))
 (segment (start 145.49 111.76) (end 146.365 111.76) (width 0.25) (layer "F.Cu") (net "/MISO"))
 (segment (start 146.177 106.649) (end 143.891 108.935) (width 0.25) (layer "F.Cu") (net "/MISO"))
 (via (at 149.86 115.634) (size 0.6) (drill 0.4) (layers "F.Cu" "B.Cu") (capping no) (covering (front no) (back no))
  (plugging (front no) (back no)) (filling no) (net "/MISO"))
 (via (at 146.177 106.553) (size 0.6) (drill 0.4) (layers "F.Cu" "B.Cu") (capping no) (covering (front no) (back no))
  (plugging (front no) (back no)) (filling no) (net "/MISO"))
 (segment (start 146.431 106.807) (end 146.177 106.553) (width 0.25) (layer "B.Cu") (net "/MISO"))
 (segment (start 149.86 105.41) (end 148.463 106.807) (width 0.25) (layer "B.Cu") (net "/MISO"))
 (segment (start 149.86 118.083) (end 149.86 115.634) (width 0.25) (layer "B.Cu") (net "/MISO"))
 (segment (start 148.463 106.807) (end 146.431 106.807) (width 0.25) (layer "B.Cu") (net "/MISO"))
 (segment (start 150.241 107.442) (end 145.542 107.442) (width 0.25) (layer "B.Cu") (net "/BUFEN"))
 (segment (start 156.083 110.871) (end 156.083 104.775) (width 0.25) (layer "B.Cu") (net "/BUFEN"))
 (segment (start 149.86 111.533) (end 151.13 111.533) (width 0.25) (layer "B.Cu") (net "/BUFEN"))
 (segment (start 143.209 109.775) (end 142.24 109.775) (width 0.25) (layer "B.Cu") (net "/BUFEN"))
 (segment (start 149.352 110.363) (end 149.86 110.871) (width 0.25) (layer "B.Cu") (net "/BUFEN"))
 (segment (start 147.32 118.083) (end 146.05 118.083) (width 0.25) (layer "B.Cu") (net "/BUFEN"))
 (segment (start 151.13 104.14) (end 151.13 106.553) (width 0.25) (layer "B.Cu") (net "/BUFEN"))
 (segment (start 151.13 106.553) (end 150.241 107.442) (width 0.25) (layer "B.Cu") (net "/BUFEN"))
 (segment (start 146.685 116.526) (end 146.685 110.617) (width 0.25) (layer "B.Cu") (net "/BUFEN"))
 (segment (start 156.083 104.775) (end 154.178 102.87) (width 0.25) (layer "B.Cu") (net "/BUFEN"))
 (segment (start 152.4 102.87) (end 151.13 104.14) (width 0.25) (layer "B.Cu") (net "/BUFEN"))
 (segment (start 149.86 110.871) (end 149.86 111.533) (width 0.25) (layer "B.Cu") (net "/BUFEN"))
 (segment (start 154.178 102.87) (end 152.4 102.87) (width 0.25) (layer "B.Cu") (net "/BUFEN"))
 (segment (start 145.542 107.442) (end 143.209 109.775) (width 0.25) (layer "B.Cu") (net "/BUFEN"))
 (segment (start 147.32 118.083) (end 147.32 117.162) (width 0.25) (layer "B.Cu") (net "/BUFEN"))
 (segment (start 151.638 110.363) (end 153.162 110.363) (width 0.25) (layer "B.Cu") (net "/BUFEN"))
 (segment (start 155.829 111.125) (end 156.083 110.871) (width 0.25) (layer "B.Cu") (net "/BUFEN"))
 (segment (start 146.685 110.617) (end 146.939 110.363) (width 0.25) (layer "B.Cu") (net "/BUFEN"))
 (segment (start 153.162 110.363) (end 153.924 111.125) (width 0.25) (layer "B.Cu") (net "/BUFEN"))
 (segment (start 153.924 111.125) (end 155.829 111.125) (width 0.25) (layer "B.Cu") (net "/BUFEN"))
 (segment (start 146.939 110.363) (end 149.352 110.363) (width 0.25) (layer "B.Cu") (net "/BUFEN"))
 (segment (start 147.32 117.162) (end 146.685 116.526) (width 0.25) (layer "B.Cu") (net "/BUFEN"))
 (segment (start 151.13 110.871) (end 151.638 110.363) (width 0.25) (layer "B.Cu") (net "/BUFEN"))
 (segment (start 151.13 111.533) (end 151.13 110.871) (width 0.25) (layer "B.Cu") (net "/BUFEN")))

